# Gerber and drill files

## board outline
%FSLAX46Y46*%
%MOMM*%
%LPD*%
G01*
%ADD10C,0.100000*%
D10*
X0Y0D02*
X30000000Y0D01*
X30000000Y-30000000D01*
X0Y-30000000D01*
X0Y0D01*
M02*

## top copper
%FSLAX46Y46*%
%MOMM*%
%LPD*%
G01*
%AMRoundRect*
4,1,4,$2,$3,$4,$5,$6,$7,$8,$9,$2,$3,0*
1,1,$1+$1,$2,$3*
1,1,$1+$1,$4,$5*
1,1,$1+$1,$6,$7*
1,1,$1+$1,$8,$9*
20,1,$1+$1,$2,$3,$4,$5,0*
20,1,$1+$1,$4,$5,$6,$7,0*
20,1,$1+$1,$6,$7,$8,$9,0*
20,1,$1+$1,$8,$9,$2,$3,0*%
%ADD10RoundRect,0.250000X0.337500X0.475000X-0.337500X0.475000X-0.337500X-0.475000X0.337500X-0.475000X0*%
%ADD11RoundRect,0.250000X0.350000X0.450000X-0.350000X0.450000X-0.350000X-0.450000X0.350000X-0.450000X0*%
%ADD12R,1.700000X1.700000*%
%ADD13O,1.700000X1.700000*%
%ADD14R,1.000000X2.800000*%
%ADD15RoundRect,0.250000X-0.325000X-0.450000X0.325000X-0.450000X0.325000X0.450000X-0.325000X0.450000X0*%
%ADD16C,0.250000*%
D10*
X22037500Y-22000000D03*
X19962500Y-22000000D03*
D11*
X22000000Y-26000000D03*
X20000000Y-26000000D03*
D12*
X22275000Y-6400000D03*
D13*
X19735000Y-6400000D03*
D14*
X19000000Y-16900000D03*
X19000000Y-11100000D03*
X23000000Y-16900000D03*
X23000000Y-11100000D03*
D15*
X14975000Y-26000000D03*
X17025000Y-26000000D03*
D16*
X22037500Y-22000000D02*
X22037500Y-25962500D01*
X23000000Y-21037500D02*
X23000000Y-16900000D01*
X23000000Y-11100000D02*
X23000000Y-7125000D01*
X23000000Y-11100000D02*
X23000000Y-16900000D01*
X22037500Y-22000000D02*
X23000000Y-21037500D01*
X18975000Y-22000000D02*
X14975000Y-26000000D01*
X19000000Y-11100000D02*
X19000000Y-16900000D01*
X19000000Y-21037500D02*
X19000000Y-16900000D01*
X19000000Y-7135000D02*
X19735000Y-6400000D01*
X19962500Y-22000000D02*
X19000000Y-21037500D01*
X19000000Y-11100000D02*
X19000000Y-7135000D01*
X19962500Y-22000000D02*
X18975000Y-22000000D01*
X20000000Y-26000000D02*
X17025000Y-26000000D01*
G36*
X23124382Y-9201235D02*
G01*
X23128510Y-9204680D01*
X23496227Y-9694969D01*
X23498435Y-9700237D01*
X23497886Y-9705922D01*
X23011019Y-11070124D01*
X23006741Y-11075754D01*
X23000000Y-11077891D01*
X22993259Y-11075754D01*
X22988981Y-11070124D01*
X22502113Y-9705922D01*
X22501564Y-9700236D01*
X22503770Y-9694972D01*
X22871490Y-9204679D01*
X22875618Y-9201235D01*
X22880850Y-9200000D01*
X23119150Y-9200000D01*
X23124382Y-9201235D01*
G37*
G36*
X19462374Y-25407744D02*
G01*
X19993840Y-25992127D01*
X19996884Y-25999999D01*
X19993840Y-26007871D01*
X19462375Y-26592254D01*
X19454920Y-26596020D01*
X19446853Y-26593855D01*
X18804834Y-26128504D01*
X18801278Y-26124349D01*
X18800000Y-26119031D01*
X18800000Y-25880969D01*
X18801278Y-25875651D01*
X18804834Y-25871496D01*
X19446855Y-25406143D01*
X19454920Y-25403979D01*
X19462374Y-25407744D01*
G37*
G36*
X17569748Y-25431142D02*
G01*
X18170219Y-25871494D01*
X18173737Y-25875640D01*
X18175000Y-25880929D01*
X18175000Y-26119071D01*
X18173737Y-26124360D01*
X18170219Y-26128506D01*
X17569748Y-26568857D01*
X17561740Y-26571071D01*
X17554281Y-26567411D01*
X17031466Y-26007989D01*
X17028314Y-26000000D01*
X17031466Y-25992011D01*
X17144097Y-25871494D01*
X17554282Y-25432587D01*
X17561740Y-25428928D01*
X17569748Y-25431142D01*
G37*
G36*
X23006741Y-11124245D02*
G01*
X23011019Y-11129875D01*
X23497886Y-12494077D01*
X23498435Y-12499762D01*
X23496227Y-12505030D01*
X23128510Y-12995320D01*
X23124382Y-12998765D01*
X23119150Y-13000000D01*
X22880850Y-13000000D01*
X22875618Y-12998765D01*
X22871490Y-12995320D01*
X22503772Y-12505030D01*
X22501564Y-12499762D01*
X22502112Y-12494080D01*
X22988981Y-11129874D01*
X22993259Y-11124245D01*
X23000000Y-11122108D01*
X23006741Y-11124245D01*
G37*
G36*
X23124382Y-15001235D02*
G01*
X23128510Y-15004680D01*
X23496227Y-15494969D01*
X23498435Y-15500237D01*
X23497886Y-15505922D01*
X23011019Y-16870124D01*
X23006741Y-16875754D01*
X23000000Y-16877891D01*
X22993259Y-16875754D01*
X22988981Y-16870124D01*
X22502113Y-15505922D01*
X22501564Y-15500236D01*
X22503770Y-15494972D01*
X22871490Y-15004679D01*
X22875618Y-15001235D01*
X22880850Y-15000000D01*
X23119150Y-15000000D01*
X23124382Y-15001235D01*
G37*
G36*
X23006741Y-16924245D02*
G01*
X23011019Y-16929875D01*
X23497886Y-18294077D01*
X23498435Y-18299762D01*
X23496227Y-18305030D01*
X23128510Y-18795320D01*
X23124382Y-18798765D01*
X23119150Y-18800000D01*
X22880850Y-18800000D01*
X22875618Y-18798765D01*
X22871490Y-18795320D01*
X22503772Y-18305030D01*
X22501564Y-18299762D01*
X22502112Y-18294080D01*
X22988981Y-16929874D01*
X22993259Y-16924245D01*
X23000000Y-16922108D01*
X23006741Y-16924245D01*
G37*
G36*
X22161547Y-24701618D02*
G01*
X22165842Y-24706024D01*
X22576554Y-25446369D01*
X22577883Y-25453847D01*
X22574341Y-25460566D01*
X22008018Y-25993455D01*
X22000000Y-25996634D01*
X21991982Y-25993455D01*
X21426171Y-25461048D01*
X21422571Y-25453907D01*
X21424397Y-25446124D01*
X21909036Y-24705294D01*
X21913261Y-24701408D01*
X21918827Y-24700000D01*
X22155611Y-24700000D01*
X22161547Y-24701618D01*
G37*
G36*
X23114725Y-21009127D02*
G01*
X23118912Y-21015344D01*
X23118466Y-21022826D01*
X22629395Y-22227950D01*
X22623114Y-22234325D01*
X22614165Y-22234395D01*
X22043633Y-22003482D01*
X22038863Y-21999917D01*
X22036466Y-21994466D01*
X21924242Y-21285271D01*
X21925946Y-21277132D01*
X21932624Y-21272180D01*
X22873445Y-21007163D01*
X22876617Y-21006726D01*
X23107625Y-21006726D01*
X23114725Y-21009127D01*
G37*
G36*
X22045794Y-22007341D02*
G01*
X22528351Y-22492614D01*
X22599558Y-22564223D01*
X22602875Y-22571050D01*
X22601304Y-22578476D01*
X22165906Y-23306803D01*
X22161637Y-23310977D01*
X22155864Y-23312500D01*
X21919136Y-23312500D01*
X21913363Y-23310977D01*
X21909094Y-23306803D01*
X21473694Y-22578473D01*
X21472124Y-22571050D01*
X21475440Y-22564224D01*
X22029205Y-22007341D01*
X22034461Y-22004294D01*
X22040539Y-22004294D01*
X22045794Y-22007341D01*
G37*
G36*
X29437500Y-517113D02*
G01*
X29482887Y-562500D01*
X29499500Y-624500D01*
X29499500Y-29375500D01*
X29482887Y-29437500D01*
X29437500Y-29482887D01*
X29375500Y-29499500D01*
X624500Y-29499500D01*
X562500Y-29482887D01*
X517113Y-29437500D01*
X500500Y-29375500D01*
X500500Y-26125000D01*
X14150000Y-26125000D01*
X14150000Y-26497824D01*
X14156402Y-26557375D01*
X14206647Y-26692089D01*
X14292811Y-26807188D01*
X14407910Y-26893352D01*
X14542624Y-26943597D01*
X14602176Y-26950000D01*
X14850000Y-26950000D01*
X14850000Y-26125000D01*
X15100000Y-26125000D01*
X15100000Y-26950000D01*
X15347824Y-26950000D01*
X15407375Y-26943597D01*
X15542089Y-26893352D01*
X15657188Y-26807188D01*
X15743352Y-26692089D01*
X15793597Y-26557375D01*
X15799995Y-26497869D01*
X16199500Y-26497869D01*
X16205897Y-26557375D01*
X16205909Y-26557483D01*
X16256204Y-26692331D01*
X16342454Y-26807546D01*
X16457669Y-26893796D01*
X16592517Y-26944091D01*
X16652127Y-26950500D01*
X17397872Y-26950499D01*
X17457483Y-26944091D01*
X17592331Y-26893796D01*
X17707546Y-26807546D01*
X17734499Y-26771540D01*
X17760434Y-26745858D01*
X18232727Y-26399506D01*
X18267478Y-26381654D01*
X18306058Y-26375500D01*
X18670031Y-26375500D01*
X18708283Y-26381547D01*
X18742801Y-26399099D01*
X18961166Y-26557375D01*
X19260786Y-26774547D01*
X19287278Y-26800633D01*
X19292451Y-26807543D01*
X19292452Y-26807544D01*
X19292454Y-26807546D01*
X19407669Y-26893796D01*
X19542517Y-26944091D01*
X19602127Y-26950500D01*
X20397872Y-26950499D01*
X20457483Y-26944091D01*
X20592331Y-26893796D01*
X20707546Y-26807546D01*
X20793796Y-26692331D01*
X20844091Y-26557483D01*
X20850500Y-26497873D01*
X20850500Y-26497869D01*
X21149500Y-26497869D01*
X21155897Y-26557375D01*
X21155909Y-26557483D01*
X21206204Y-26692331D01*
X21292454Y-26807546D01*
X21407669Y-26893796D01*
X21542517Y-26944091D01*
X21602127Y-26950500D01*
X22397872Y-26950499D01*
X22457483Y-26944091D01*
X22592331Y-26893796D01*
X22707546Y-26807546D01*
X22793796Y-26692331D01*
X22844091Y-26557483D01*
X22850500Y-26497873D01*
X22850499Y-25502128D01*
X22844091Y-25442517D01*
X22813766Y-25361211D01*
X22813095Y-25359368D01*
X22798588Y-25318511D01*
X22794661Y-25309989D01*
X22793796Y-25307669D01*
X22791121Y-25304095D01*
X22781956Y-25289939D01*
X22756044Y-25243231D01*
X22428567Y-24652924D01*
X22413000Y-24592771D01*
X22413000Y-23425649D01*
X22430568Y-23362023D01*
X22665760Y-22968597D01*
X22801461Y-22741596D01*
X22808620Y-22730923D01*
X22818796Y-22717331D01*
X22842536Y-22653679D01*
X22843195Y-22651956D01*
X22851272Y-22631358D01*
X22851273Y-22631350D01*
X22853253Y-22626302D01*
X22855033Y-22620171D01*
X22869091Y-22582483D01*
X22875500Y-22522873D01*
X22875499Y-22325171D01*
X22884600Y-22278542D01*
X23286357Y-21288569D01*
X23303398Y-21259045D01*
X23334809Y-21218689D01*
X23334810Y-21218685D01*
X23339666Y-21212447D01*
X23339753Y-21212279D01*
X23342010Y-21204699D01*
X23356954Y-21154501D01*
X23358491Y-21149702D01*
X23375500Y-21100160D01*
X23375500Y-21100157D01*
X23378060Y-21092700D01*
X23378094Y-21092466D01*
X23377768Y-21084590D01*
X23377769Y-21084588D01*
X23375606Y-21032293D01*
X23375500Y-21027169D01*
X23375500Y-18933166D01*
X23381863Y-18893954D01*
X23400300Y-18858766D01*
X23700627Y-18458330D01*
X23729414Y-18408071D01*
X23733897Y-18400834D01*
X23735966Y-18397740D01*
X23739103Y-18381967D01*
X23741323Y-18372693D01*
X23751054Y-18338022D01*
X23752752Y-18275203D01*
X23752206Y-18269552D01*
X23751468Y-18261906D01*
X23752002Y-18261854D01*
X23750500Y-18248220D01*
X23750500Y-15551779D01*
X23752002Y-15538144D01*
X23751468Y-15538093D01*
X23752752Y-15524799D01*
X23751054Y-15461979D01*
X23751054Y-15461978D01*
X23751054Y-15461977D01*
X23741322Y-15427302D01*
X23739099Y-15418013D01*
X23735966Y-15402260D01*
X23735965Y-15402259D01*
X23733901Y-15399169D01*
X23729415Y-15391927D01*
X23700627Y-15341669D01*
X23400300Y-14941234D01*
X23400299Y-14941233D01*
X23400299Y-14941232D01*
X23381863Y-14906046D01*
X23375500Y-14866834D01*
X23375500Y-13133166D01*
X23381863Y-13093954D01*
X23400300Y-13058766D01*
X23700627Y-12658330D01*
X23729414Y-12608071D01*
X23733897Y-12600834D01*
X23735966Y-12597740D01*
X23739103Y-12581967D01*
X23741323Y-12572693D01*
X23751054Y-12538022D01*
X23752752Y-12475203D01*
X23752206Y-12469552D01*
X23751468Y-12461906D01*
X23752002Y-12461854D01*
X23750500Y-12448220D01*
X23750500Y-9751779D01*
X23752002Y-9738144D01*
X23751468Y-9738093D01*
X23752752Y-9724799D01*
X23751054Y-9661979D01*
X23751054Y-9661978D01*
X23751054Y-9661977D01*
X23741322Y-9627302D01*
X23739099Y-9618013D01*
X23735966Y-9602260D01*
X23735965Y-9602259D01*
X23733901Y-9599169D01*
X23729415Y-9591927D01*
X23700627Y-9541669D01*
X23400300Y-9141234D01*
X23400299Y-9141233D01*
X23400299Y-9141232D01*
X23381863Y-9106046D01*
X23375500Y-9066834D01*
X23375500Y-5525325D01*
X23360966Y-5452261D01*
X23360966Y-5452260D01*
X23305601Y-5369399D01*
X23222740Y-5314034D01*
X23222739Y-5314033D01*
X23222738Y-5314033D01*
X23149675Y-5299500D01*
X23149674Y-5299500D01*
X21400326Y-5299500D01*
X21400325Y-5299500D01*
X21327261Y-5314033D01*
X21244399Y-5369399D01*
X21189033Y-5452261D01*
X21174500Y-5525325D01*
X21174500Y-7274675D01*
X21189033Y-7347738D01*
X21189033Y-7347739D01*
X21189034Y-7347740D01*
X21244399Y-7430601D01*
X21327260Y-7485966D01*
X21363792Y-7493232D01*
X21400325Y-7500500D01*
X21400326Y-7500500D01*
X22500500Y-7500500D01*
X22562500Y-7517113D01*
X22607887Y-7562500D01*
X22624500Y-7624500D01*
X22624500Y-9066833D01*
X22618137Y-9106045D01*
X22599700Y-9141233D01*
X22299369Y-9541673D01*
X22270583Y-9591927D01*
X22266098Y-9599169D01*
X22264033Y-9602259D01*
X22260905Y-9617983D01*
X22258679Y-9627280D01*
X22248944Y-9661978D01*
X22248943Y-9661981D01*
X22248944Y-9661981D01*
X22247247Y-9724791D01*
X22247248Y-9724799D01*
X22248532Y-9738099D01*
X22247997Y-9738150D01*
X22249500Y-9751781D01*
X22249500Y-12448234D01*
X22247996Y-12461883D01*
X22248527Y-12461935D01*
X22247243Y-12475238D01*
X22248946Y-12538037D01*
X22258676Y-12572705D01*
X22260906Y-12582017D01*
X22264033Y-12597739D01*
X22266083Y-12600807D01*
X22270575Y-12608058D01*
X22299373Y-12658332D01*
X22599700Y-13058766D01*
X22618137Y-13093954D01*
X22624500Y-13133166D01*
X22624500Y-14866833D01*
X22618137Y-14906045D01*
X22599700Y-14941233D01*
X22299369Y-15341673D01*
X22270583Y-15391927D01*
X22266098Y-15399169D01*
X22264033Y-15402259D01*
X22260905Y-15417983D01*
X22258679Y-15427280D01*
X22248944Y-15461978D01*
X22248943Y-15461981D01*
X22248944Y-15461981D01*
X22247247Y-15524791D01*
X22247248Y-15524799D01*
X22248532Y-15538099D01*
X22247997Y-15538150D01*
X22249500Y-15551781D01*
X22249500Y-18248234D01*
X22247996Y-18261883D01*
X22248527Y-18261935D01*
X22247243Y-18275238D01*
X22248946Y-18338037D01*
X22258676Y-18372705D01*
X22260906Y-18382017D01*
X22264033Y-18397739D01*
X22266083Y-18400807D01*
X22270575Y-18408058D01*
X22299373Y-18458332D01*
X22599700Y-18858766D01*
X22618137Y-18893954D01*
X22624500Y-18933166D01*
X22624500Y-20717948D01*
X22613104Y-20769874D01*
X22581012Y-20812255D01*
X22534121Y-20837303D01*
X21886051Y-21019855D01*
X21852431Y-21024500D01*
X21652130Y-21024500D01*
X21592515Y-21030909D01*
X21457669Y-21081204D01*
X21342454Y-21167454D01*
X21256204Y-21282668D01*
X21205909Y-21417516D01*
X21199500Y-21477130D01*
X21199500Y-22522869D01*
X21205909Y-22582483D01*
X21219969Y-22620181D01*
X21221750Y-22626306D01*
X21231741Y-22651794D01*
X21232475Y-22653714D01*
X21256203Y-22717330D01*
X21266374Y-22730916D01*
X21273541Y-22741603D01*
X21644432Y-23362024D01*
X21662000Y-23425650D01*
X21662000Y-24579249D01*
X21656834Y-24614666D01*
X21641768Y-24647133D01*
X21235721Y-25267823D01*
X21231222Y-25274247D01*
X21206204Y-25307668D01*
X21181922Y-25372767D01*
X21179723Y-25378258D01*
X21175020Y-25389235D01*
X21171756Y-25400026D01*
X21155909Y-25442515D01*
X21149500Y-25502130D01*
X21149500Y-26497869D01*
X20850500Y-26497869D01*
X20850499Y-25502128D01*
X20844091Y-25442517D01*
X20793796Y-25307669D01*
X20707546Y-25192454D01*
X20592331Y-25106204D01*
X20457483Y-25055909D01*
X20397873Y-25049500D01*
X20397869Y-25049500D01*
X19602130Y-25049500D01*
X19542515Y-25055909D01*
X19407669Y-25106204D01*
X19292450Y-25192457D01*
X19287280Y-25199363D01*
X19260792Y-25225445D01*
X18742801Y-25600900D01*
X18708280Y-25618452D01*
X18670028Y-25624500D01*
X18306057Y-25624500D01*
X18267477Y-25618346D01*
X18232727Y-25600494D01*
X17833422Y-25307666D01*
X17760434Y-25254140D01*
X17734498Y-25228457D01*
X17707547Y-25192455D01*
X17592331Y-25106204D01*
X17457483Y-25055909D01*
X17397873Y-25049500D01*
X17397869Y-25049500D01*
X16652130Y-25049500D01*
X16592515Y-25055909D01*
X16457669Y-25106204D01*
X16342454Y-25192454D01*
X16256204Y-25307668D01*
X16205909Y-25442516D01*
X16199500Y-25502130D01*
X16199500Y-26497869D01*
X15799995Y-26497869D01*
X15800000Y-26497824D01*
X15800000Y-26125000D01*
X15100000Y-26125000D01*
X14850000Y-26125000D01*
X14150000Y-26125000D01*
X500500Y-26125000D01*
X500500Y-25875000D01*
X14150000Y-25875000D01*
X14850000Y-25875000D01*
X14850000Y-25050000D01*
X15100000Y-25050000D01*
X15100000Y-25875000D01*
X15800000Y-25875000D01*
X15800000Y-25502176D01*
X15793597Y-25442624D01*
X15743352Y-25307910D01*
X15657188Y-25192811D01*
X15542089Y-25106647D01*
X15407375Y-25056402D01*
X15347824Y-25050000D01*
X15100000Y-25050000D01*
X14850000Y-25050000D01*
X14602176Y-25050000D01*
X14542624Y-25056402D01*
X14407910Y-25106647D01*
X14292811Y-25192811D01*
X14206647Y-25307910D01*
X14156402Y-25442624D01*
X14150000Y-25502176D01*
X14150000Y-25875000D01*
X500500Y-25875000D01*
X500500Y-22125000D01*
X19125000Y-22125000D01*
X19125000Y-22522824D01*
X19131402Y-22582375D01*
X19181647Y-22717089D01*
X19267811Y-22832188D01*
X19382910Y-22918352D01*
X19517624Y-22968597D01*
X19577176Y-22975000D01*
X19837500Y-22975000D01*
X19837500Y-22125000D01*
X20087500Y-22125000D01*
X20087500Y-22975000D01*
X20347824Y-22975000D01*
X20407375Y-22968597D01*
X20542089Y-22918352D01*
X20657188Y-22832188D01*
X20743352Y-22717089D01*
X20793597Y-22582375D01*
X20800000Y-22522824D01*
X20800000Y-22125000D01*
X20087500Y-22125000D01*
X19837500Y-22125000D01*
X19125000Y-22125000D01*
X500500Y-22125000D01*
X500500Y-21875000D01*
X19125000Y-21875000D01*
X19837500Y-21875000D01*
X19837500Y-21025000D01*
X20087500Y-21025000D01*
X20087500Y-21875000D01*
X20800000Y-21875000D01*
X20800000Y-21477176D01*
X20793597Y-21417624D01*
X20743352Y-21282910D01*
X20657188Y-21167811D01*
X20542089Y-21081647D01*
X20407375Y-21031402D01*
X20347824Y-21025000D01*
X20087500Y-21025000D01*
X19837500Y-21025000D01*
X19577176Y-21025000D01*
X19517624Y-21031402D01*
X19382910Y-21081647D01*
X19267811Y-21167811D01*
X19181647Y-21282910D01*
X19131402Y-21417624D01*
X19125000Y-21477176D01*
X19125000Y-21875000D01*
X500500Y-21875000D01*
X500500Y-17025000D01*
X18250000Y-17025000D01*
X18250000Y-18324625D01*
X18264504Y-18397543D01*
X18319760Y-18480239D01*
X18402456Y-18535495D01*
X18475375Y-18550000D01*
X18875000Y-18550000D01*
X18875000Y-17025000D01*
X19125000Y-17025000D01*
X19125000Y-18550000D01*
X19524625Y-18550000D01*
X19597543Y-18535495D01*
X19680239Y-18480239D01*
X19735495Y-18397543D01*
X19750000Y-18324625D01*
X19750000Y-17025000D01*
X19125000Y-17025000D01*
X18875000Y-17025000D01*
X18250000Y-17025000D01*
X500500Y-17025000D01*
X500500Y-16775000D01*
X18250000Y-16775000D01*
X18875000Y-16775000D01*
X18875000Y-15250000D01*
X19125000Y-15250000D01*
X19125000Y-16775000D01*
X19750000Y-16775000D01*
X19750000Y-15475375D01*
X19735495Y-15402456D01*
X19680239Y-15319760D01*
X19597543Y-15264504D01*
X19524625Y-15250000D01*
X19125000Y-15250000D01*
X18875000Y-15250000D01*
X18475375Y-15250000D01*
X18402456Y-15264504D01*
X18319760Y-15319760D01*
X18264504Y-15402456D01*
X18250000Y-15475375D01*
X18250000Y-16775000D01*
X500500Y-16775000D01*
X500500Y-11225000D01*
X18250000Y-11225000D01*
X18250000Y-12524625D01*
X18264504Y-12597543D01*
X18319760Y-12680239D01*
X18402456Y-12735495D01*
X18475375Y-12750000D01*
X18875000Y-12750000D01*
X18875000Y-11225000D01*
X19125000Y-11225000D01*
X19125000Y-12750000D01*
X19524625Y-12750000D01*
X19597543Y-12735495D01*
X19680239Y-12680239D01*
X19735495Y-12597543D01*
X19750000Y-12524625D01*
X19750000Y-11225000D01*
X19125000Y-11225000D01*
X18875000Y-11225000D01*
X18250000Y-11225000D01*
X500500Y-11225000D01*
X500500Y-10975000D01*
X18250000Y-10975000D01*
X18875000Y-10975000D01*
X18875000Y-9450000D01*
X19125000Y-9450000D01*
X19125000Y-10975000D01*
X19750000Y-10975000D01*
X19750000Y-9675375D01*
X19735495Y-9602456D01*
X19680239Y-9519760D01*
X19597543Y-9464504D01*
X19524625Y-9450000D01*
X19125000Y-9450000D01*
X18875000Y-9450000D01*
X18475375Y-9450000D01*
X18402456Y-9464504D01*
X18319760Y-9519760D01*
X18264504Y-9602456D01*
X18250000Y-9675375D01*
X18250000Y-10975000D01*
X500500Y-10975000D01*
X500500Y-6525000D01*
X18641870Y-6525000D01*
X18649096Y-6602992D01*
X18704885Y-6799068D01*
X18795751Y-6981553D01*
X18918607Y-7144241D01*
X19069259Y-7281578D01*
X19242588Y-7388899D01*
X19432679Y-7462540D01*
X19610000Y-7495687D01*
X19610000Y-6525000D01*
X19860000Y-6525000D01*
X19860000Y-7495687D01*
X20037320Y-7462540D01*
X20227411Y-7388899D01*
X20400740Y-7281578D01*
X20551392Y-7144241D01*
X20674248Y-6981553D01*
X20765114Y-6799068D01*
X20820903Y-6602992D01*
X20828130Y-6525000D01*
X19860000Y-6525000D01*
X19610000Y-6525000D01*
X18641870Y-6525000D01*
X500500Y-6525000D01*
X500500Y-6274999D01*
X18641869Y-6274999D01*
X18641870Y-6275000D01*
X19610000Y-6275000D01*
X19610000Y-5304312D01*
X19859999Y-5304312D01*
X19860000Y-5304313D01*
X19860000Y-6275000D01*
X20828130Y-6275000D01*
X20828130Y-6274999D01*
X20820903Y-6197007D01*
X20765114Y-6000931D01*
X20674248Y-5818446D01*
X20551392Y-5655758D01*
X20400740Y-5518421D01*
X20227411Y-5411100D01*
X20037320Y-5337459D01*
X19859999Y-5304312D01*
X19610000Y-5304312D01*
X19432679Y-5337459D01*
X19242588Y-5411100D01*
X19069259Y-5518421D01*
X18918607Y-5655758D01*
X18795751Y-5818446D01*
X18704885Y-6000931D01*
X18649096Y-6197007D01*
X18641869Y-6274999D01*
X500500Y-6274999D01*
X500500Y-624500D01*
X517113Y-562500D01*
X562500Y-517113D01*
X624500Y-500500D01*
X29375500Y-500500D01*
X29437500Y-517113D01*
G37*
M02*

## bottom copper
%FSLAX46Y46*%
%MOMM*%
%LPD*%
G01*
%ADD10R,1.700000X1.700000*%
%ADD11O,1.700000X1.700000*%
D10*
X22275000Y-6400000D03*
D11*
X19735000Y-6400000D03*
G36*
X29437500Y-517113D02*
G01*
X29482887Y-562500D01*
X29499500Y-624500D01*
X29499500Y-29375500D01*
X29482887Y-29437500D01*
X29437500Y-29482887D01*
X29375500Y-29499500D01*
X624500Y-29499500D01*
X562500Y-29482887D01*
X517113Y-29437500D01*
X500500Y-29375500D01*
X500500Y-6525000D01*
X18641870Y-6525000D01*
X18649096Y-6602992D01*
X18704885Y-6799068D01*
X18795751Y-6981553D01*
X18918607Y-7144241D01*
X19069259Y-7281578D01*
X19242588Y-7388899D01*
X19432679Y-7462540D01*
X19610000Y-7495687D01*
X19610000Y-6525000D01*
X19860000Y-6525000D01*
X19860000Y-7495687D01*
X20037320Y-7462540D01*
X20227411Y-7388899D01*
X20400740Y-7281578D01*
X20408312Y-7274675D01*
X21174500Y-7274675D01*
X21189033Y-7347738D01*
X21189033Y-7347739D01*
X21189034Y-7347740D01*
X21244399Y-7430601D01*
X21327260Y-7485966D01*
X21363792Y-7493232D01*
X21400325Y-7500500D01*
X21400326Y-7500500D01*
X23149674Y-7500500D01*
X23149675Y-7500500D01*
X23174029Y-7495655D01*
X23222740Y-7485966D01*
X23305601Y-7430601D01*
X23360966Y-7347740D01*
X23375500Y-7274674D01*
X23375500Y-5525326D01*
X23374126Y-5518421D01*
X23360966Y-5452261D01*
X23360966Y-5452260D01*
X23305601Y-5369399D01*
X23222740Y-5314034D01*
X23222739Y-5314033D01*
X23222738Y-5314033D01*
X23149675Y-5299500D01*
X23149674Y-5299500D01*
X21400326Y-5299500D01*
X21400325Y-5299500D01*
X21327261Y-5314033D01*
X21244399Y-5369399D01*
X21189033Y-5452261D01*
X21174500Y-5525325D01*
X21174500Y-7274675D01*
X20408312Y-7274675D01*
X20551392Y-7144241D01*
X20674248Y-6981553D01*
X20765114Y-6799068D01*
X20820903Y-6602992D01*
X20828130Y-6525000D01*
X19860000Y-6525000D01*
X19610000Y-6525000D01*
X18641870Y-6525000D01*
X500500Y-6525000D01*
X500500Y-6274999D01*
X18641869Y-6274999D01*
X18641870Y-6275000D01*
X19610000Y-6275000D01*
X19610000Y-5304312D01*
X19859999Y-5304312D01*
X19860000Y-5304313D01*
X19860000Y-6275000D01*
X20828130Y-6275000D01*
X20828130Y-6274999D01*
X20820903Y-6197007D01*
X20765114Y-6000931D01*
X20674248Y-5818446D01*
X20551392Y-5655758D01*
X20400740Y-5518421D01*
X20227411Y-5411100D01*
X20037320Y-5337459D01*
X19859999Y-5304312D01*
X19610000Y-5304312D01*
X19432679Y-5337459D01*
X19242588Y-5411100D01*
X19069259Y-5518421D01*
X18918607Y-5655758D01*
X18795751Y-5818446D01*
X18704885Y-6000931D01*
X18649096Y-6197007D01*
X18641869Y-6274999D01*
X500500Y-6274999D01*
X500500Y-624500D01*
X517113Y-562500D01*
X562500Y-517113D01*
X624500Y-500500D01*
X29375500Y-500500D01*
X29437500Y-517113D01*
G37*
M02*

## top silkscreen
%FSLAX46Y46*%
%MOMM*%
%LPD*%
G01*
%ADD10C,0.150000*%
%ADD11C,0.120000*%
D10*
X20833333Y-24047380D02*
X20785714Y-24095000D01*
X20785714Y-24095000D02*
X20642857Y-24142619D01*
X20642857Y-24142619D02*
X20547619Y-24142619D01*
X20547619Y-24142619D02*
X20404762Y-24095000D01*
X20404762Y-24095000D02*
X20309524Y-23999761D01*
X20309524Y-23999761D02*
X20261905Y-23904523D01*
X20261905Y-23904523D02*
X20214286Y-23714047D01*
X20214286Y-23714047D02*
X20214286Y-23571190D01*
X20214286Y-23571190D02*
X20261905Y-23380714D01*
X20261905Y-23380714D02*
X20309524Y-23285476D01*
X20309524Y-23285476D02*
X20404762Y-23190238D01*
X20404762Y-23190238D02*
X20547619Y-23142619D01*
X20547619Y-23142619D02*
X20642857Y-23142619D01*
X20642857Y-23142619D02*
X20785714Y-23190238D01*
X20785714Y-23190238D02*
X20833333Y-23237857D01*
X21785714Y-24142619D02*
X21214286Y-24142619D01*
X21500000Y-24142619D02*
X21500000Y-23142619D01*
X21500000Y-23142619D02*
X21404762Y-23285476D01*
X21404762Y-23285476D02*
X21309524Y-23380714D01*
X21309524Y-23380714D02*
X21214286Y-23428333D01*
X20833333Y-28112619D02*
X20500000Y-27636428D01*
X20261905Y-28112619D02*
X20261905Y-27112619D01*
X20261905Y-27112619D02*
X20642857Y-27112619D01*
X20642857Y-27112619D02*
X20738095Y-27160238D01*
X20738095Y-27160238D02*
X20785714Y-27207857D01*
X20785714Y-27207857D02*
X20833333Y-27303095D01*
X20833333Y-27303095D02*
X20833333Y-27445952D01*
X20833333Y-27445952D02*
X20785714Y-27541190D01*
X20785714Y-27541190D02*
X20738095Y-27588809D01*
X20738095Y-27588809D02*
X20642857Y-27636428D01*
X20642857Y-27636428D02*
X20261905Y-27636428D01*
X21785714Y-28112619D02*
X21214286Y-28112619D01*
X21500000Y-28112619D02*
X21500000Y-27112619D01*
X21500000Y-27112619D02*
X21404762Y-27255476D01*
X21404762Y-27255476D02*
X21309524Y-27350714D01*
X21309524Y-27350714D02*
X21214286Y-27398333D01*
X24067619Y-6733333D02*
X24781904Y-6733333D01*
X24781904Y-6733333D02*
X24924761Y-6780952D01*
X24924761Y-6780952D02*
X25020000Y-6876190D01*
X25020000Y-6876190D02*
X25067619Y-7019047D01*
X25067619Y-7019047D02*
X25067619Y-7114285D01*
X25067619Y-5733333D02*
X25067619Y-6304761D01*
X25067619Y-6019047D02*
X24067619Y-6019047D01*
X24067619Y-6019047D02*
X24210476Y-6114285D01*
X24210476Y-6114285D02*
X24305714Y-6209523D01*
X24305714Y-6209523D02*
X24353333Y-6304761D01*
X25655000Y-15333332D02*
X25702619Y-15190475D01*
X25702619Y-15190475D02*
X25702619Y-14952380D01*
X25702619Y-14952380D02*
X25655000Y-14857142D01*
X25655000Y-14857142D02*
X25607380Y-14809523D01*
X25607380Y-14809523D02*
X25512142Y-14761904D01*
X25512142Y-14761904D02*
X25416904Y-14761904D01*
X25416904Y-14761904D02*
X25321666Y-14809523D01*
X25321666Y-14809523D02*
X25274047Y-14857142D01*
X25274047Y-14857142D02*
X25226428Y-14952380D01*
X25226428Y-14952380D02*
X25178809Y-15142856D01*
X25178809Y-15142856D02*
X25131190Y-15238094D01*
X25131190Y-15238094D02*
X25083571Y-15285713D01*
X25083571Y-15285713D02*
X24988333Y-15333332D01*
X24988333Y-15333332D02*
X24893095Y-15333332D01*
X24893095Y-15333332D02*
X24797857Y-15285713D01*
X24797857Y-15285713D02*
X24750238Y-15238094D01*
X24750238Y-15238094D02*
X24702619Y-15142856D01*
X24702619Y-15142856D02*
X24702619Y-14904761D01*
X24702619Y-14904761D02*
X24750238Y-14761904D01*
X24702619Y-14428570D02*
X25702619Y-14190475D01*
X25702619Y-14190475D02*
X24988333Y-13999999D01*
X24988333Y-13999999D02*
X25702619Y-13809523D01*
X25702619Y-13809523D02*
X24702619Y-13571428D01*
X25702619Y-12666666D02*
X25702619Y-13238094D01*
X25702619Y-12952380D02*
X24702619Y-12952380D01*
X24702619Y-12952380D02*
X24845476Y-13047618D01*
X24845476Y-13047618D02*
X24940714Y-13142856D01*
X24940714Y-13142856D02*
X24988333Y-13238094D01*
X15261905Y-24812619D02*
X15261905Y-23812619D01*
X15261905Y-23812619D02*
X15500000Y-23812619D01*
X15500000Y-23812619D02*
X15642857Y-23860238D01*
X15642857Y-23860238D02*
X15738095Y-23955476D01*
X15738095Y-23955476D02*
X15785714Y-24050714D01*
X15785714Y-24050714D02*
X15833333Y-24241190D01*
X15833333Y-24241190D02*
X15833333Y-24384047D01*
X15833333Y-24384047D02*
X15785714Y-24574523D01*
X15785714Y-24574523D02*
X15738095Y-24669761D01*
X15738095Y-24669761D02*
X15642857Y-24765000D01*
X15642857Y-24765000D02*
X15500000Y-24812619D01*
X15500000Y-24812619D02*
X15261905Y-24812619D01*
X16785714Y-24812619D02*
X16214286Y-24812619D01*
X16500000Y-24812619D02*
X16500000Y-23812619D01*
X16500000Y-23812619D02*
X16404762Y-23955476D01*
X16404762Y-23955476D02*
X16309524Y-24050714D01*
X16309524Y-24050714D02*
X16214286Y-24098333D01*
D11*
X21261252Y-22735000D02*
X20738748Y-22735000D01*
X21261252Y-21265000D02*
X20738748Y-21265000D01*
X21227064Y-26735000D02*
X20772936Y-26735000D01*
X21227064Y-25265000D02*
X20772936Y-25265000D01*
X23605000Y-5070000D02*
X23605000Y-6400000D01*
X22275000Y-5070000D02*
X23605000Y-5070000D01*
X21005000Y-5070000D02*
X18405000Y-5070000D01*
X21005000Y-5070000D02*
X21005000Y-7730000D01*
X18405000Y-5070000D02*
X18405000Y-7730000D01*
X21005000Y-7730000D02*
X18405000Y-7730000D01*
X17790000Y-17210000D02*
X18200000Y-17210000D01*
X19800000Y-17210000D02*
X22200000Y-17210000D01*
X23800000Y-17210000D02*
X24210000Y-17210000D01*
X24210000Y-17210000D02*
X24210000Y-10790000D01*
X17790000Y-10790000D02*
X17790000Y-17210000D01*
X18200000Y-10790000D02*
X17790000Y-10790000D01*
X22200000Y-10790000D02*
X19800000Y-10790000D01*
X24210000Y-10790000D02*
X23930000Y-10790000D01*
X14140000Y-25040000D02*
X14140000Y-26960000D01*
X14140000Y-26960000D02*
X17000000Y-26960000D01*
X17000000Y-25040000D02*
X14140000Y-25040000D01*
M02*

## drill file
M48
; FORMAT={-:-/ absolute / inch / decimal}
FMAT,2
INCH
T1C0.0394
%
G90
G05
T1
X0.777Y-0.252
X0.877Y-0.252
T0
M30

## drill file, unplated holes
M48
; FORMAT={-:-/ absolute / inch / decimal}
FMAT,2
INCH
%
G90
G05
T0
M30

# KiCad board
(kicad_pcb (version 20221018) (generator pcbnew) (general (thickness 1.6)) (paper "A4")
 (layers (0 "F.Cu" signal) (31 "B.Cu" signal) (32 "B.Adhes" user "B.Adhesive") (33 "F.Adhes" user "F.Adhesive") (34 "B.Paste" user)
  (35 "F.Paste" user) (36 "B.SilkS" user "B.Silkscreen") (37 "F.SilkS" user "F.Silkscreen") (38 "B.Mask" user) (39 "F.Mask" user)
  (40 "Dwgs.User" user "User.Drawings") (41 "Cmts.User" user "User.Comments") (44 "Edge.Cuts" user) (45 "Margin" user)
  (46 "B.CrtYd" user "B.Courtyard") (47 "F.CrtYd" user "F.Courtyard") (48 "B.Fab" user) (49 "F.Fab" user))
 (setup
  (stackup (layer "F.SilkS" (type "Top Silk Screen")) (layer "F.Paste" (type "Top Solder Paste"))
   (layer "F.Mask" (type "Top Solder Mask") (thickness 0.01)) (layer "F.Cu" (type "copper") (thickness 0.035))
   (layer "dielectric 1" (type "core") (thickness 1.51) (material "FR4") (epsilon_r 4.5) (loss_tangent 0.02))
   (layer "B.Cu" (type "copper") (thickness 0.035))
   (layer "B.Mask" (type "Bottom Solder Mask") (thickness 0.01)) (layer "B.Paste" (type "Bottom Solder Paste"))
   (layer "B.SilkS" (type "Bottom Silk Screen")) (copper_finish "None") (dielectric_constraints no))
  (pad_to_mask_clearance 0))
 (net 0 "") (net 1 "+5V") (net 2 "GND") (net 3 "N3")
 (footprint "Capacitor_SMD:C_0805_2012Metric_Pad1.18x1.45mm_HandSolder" (layer "F.Cu") (at 21 22 180)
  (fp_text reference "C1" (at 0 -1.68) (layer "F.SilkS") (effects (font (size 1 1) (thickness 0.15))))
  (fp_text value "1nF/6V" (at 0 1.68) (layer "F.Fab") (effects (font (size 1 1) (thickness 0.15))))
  (fp_line (start -0.261252 -0.735) (end 0.261252 -0.735) (stroke (width 0.12) (type solid)) (layer "F.SilkS"))
  (fp_line (start -0.261252 0.735) (end 0.261252 0.735) (stroke (width 0.12) (type solid)) (layer "F.SilkS"))
  (pad "1" smd roundrect (at -1.0375 0 180) (size 1.175 1.45) (layers "F.Cu" "F.Paste" "F.Mask") (roundrect_rratio 0.2127659574)
   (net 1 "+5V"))
  (pad "2" smd roundrect (at 1.0375 0 180) (size 1.175 1.45) (layers "F.Cu" "F.Paste" "F.Mask") (roundrect_rratio 0.2127659574)
   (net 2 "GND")))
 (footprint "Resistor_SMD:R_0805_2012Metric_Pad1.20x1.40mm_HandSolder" (layer "F.Cu") (at 21 26 180)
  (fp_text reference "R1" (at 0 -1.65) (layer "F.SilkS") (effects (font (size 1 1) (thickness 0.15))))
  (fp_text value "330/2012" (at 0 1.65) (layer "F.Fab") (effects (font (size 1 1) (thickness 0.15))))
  (fp_line (start -0.227064 -0.735) (end 0.227064 -0.735) (stroke (width 0.12) (type solid)) (layer "F.SilkS"))
  (fp_line (start -0.227064 0.735) (end 0.227064 0.735) (stroke (width 0.12) (type solid)) (layer "F.SilkS"))
  (pad "1" smd roundrect (at -1 0 180) (size 1.2 1.4) (layers "F.Cu" "F.Paste" "F.Mask") (roundrect_rratio 0.2083333333) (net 1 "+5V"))
  (pad "2" smd roundrect (at 1 0 180) (size 1.2 1.4) (layers "F.Cu" "F.Paste" "F.Mask") (roundrect_rratio 0.2083333333) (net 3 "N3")))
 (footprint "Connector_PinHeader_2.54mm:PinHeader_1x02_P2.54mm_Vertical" (layer "F.Cu") (at 22.275 6.4 -90)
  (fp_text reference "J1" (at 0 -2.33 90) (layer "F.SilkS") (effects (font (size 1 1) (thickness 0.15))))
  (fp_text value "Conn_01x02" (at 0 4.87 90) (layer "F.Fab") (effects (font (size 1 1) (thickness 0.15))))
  (fp_line (start -1.33 -1.33) (end 0 -1.33) (stroke (width 0.12) (type solid)) (layer "F.SilkS"))
  (fp_line (start -1.33 0) (end -1.33 -1.33) (stroke (width 0.12) (type solid)) (layer "F.SilkS"))
  (fp_line (start -1.33 1.27) (end -1.33 3.87) (stroke (width 0.12) (type solid)) (layer "F.SilkS"))
  (fp_line (start -1.33 1.27) (end 1.33 1.27) (stroke (width 0.12) (type solid)) (layer "F.SilkS"))
  (fp_line (start -1.33 3.87) (end 1.33 3.87) (stroke (width 0.12) (type solid)) (layer "F.SilkS"))
  (fp_line (start 1.33 1.27) (end 1.33 3.87) (stroke (width 0.12) (type solid)) (layer "F.SilkS"))
  (pad "1" thru_hole rect (at 0 0 270) (size 1.7 1.7) (drill 1) (layers "*.Cu" "*.Mask") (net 1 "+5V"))
  (pad "2" thru_hole oval (at 0 2.54 270) (size 1.7 1.7) (drill 1) (layers "*.Cu" "*.Mask") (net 2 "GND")))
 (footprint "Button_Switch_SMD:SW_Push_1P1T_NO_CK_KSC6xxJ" (layer "F.Cu") (at 21 14 90)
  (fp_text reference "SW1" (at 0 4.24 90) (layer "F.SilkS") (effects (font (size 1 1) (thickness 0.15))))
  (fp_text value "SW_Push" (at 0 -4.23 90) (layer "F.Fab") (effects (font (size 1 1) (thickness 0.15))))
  (fp_line (start -3.21 -3.21) (end -3.21 -2.8) (stroke (width 0.12) (type solid)) (layer "F.SilkS"))
  (fp_line (start -3.21 -1.2) (end -3.21 1.2) (stroke (width 0.12) (type solid)) (layer "F.SilkS"))
  (fp_line (start -3.21 2.8) (end -3.21 3.21) (stroke (width 0.12) (type solid)) (layer "F.SilkS"))
  (fp_line (start -3.21 3.21) (end 3.21 3.21) (stroke (width 0.12) (type solid)) (layer "F.SilkS"))
  (fp_line (start 3.21 -3.21) (end -3.21 -3.21) (stroke (width 0.12) (type solid)) (layer "F.SilkS"))
  (fp_line (start 3.21 -2.8) (end 3.21 -3.21) (stroke (width 0.12) (type solid)) (layer "F.SilkS"))
  (fp_line (start 3.21 1.2) (end 3.21 -1.2) (stroke (width 0.12) (type solid)) (layer "F.SilkS"))
  (fp_line (start 3.21 3.21) (end 3.21 2.93) (stroke (width 0.12) (type solid)) (layer "F.SilkS"))
  (pad "1" smd rect (at -2.9 -2 90) (size 2.8 1) (layers "F.Cu" "F.Paste" "F.Mask") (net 2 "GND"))
  (pad "1" smd rect (at 2.9 -2 90) (size 2.8 1) (layers "F.Cu" "F.Paste" "F.Mask") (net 2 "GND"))
  (pad "2" smd rect (at -2.9 2 90) (size 2.8 1) (layers "F.Cu" "F.Paste" "F.Mask") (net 1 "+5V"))
  (pad "2" smd rect (at 2.9 2 90) (size 2.8 1) (layers "F.Cu" "F.Paste" "F.Mask") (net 1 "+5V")))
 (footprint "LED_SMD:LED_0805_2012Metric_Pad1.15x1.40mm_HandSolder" (layer "F.Cu") (at 16 26)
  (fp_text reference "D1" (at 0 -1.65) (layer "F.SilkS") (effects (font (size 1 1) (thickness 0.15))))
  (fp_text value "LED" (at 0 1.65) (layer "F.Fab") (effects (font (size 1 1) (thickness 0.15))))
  (fp_line (start -1.86 -0.96) (end -1.86 0.96) (stroke (width 0.12) (type solid)) (layer "F.SilkS"))
  (fp_line (start -1.86 0.96) (end 1 0.96) (stroke (width 0.12) (type solid)) (layer "F.SilkS"))
  (fp_line (start 1 -0.96) (end -1.86 -0.96) (stroke (width 0.12) (type solid)) (layer "F.SilkS"))
  (pad "1" smd roundrect (at -1.025 0) (size 1.15 1.4) (layers "F.Cu" "F.Paste" "F.Mask") (roundrect_rratio 0.2173913043) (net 2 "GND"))
  (pad "2" smd roundrect (at 1.025 0) (size 1.15 1.4) (layers "F.Cu" "F.Paste" "F.Mask") (roundrect_rratio 0.2173913043) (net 3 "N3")))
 (gr_rect locked (start 0 0) (end 30 30) (stroke (width 0.1) (type default)) (fill none) (layer "Edge.Cuts"))
 (segment (start 22.0375 22) (end 22.0375 25.9625) (width 0.25) (layer "F.Cu") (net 1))
 (segment (start 23 21.0375) (end 23 16.9) (width 0.25) (layer "F.Cu") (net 1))
 (segment (start 23 11.1) (end 23 7.125) (width 0.25) (layer "F.Cu") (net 1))
 (segment (start 23 11.1) (end 23 16.9) (width 0.25) (layer "F.Cu") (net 1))
 (segment (start 22.0375 22) (end 23 21.0375) (width 0.25) (layer "F.Cu") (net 1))
 (segment (start 18.975 22) (end 14.975 26) (width 0.25) (layer "F.Cu") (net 2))
 (segment (start 19 11.1) (end 19 16.9) (width 0.25) (layer "F.Cu") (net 2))
 (segment (start 19 21.0375) (end 19 16.9) (width 0.25) (layer "F.Cu") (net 2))
 (segment (start 19 7.135) (end 19.735 6.4) (width 0.25) (layer "F.Cu") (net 2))
 (segment (start 19.9625 22) (end 19 21.0375) (width 0.25) (layer "F.Cu") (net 2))
 (segment (start 19 11.1) (end 19 7.135) (width 0.25) (layer "F.Cu") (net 2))
 (segment (start 19.9625 22) (end 18.975 22) (width 0.25) (layer "F.Cu") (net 2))
 (segment (start 20 26) (end 17.025 26) (width 0.25) (layer "F.Cu") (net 3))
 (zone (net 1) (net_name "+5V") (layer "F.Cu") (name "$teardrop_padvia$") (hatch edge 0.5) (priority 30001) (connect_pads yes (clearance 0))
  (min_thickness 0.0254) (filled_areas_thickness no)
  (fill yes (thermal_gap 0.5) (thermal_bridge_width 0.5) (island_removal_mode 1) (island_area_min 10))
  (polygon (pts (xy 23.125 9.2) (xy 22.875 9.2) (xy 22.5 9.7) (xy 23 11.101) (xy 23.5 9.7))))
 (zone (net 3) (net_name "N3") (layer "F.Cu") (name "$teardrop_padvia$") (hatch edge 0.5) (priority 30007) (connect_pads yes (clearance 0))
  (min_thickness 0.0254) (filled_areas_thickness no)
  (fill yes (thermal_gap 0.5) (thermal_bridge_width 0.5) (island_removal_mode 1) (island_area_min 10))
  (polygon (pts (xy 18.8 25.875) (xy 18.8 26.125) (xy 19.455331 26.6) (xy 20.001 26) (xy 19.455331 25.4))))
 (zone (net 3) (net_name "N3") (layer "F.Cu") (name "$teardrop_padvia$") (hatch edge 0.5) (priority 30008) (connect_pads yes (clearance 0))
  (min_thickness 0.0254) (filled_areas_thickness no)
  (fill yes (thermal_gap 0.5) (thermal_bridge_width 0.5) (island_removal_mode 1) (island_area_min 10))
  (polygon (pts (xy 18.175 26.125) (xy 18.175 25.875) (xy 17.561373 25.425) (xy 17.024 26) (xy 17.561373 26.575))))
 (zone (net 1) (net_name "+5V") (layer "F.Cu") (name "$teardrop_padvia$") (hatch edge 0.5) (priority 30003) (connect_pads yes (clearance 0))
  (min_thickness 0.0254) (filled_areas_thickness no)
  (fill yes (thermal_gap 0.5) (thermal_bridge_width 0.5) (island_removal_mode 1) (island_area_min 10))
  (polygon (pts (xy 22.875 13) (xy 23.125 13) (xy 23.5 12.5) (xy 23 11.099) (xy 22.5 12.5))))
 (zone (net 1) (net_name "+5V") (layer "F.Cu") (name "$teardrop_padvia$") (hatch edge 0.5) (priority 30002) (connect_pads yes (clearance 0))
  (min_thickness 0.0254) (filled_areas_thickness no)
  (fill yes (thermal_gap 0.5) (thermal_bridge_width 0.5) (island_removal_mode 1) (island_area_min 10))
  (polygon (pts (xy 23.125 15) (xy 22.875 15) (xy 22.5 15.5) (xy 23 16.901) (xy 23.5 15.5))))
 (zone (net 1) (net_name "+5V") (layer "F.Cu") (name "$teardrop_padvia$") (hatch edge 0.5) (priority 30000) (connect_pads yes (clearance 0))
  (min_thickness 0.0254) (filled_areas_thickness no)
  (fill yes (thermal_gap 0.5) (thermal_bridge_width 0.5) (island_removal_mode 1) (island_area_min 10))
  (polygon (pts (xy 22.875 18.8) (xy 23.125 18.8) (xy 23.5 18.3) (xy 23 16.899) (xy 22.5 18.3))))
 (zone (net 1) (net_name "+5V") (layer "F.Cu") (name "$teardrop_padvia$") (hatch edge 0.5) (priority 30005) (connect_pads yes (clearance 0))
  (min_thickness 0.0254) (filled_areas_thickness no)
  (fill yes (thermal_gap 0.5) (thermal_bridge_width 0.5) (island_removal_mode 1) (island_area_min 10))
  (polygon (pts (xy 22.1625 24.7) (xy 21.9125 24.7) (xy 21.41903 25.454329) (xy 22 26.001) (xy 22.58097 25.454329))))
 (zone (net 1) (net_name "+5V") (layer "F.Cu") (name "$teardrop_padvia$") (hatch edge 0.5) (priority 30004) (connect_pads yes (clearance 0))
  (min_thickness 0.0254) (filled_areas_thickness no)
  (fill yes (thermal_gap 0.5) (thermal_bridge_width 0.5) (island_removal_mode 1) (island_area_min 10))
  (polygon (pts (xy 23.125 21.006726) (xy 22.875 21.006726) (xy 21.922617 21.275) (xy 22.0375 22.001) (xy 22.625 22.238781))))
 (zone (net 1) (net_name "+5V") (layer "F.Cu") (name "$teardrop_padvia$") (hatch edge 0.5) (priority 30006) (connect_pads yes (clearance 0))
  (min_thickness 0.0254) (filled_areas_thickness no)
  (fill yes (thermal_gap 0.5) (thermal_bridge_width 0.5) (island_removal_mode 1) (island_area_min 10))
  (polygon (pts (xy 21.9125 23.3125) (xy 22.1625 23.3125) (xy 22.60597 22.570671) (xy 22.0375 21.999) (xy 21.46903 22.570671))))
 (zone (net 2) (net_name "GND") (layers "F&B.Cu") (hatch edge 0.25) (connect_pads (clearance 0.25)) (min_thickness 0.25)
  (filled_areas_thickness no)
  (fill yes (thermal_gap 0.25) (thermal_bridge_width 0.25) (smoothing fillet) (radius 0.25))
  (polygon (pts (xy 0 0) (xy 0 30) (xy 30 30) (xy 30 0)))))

